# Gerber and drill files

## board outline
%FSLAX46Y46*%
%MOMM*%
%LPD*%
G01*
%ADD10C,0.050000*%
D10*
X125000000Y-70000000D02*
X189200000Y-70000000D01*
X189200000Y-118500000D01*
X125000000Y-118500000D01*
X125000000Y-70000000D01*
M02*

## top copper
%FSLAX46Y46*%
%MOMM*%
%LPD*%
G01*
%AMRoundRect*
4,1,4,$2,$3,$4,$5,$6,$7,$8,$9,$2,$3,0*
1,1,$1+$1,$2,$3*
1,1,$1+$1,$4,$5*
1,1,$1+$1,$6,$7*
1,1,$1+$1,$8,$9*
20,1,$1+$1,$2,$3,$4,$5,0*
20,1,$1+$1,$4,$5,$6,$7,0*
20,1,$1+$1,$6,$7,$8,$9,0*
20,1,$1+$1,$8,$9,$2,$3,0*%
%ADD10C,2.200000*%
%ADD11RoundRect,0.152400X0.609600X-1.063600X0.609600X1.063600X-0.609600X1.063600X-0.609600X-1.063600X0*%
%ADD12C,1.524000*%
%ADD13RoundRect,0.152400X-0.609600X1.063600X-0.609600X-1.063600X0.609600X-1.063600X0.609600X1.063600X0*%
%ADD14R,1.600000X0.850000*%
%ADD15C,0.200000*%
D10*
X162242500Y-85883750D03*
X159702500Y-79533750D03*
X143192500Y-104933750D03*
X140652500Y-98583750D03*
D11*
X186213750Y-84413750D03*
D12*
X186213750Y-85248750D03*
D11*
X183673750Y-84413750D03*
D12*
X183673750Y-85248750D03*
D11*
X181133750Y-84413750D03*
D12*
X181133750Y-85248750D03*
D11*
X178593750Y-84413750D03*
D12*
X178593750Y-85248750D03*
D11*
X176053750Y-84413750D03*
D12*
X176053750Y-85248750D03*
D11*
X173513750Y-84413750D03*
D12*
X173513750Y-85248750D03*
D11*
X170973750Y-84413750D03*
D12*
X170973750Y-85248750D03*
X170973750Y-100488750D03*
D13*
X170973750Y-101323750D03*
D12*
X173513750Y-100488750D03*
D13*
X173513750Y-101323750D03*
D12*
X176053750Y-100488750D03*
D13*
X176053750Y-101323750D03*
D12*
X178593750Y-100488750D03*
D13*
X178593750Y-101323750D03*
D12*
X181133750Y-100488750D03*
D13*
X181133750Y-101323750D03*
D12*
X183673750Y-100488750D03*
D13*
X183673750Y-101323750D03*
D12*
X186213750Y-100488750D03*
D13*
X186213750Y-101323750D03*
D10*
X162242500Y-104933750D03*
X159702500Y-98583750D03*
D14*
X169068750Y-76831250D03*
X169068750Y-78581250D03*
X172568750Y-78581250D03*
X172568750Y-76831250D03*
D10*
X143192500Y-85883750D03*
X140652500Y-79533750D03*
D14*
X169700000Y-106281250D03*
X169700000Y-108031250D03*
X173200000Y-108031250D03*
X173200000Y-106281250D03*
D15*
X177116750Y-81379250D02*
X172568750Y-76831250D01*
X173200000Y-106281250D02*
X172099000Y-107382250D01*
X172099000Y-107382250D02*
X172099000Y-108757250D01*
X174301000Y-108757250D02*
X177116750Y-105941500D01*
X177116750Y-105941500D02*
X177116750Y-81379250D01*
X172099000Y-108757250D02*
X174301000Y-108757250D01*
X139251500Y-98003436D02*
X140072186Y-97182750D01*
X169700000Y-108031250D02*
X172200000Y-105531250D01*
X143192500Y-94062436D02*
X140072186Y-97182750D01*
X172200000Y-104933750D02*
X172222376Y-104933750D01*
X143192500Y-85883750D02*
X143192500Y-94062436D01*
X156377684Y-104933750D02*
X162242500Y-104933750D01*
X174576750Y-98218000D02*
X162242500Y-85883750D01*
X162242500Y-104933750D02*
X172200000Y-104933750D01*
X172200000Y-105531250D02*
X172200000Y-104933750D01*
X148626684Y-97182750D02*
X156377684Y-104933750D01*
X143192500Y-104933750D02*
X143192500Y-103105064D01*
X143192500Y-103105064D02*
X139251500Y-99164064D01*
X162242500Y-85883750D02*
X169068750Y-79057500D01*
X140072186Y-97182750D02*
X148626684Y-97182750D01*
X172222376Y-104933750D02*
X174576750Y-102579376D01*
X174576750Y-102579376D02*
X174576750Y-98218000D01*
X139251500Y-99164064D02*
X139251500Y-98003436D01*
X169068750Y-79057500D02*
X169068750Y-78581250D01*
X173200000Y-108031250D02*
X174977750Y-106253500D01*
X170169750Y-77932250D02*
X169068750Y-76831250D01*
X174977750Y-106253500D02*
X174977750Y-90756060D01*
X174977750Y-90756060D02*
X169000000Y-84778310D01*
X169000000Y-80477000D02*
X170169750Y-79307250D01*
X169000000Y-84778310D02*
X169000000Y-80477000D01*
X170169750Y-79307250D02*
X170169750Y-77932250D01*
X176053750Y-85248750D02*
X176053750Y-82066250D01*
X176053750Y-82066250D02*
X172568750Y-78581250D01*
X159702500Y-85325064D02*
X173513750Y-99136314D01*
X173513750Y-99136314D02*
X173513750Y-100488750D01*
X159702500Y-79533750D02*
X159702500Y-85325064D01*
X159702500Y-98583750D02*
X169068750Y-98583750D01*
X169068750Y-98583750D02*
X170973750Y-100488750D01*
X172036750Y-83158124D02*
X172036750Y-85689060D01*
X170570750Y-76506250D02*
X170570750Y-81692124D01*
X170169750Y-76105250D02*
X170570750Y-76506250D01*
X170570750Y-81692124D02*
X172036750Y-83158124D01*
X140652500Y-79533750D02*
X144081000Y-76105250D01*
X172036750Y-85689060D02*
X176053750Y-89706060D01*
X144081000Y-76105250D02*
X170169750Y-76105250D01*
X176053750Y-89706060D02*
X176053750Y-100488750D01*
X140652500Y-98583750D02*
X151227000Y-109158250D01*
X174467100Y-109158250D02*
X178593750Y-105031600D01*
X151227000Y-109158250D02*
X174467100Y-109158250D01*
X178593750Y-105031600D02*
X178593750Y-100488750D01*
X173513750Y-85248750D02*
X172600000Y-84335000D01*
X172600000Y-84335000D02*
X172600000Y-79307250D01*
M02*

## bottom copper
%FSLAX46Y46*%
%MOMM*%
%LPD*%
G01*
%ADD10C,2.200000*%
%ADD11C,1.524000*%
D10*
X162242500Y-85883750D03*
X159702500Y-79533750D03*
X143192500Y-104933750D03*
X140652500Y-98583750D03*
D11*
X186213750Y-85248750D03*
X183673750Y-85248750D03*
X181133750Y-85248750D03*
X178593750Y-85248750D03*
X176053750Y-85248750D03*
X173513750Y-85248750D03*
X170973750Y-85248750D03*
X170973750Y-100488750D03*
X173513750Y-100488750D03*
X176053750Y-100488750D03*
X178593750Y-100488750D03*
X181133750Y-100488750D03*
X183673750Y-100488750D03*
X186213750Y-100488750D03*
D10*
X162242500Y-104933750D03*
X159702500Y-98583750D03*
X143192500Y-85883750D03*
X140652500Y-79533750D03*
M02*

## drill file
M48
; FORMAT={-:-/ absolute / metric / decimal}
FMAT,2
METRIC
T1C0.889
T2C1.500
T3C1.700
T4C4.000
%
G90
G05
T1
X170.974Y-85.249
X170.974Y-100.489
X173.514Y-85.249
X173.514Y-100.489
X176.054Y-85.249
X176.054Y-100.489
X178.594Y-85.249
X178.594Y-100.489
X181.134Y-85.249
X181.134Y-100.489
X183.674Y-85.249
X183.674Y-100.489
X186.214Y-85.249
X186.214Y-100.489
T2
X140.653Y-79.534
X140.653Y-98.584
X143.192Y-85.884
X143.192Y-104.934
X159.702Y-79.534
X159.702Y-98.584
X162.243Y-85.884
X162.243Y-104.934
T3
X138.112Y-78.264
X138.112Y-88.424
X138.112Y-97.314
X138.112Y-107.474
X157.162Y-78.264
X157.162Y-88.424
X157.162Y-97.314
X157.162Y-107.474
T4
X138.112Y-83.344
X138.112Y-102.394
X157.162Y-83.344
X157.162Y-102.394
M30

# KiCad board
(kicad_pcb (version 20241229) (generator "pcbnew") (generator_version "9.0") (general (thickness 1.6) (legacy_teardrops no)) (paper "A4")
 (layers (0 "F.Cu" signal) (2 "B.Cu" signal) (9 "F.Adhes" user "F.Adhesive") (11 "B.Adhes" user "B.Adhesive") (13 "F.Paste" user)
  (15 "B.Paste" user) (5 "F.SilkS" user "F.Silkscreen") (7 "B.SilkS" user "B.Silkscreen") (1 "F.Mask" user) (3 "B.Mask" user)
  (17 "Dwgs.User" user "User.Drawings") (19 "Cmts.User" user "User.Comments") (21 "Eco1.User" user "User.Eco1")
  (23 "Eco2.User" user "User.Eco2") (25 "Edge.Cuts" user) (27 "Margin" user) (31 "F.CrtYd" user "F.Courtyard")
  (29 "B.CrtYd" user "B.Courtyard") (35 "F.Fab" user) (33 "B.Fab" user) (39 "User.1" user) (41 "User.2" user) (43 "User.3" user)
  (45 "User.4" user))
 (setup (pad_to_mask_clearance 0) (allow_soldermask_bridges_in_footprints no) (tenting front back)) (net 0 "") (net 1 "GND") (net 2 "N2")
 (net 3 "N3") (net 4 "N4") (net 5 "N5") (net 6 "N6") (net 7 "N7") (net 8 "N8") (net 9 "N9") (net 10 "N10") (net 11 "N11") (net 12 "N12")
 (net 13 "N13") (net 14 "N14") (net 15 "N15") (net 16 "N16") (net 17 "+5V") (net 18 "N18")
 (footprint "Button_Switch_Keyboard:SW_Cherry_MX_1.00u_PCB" (layer "F.Cu") (at 162.2425 85.88375 -90)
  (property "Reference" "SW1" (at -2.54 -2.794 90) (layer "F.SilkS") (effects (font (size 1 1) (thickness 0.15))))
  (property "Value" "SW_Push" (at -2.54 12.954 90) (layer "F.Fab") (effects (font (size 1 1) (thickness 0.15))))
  (pad "" np_thru_hole circle (at -7.62 5.08 270) (size 1.7 1.7) (drill 1.7) (layers "*.Cu" "*.Mask"))
  (pad "" np_thru_hole circle (at -2.54 5.08 270) (size 4 4) (drill 4) (layers "*.Cu" "*.Mask"))
  (pad "" np_thru_hole circle (at 2.54 5.08 270) (size 1.7 1.7) (drill 1.7) (layers "*.Cu" "*.Mask"))
  (pad "1" thru_hole circle (at 0 0 270) (size 2.2 2.2) (drill 1.5) (layers "*.Cu" "*.Mask") (remove_unused_layers no) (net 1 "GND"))
  (pad "2" thru_hole circle (at -6.35 2.54 270) (size 2.2 2.2) (drill 1.5) (layers "*.Cu" "*.Mask") (remove_unused_layers no) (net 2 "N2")))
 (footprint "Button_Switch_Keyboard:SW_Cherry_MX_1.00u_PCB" (layer "F.Cu") (at 143.1925 104.93375 -90)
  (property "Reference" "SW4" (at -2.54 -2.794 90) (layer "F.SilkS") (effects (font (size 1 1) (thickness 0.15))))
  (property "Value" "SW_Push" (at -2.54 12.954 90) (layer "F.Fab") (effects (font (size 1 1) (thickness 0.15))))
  (pad "" np_thru_hole circle (at -7.62 5.08 270) (size 1.7 1.7) (drill 1.7) (layers "*.Cu" "*.Mask"))
  (pad "" np_thru_hole circle (at -2.54 5.08 270) (size 4 4) (drill 4) (layers "*.Cu" "*.Mask"))
  (pad "" np_thru_hole circle (at 2.54 5.08 270) (size 1.7 1.7) (drill 1.7) (layers "*.Cu" "*.Mask"))
  (pad "1" thru_hole circle (at 0 0 270) (size 2.2 2.2) (drill 1.5) (layers "*.Cu" "*.Mask") (remove_unused_layers no) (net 1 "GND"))
  (pad "2" thru_hole circle (at -6.35 2.54 270) (size 2.2 2.2) (drill 1.5) (layers "*.Cu" "*.Mask") (remove_unused_layers no) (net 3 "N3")))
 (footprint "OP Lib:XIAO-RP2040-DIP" (layer "F.Cu") (at 178.59375 92.86875 -90)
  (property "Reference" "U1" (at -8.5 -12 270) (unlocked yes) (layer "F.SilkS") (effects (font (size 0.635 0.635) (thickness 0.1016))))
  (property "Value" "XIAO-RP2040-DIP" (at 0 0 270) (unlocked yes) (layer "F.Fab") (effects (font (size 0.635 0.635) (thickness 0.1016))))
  (pad "1" smd roundrect (at -8.455 -7.62 90) (size 2.432 1.524) (layers "F.Cu" "F.Mask") (roundrect_rratio 0.1) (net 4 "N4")
   (thermal_bridge_angle 45))
  (pad "1" thru_hole circle (at -7.62 -7.62 90) (size 1.524 1.524) (drill 0.889) (layers "*.Cu" "*.Mask") (remove_unused_layers no)
   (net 4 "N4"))
  (pad "2" smd roundrect (at -8.455 -5.08 90) (size 2.432 1.524) (layers "F.Cu" "F.Mask") (roundrect_rratio 0.1) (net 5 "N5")
   (thermal_bridge_angle 45))
  (pad "2" thru_hole circle (at -7.62 -5.08 90) (size 1.524 1.524) (drill 0.889) (layers "*.Cu" "*.Mask") (remove_unused_layers no)
   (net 5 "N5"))
  (pad "3" smd roundrect (at -8.455 -2.54 90) (size 2.432 1.524) (layers "F.Cu" "F.Mask") (roundrect_rratio 0.1) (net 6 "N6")
   (thermal_bridge_angle 45))
  (pad "3" thru_hole circle (at -7.62 -2.54 90) (size 1.524 1.524) (drill 0.889) (layers "*.Cu" "*.Mask") (remove_unused_layers no)
   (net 6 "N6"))
  (pad "4" smd roundrect (at -8.455 0 90) (size 2.432 1.524) (layers "F.Cu" "F.Mask") (roundrect_rratio 0.1) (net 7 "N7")
   (thermal_bridge_angle 45))
  (pad "4" thru_hole circle (at -7.62 0 90) (size 1.524 1.524) (drill 0.889) (layers "*.Cu" "*.Mask") (remove_unused_layers no) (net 7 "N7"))
  (pad "5" smd roundrect (at -8.455 2.54 90) (size 2.432 1.524) (layers "F.Cu" "F.Mask") (roundrect_rratio 0.1) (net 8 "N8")
   (thermal_bridge_angle 45))
  (pad "5" thru_hole circle (at -7.62 2.54 90) (size 1.524 1.524) (drill 0.889) (layers "*.Cu" "*.Mask") (remove_unused_layers no)
   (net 8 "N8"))
  (pad "6" smd roundrect (at -8.455 5.08 90) (size 2.432 1.524) (layers "F.Cu" "F.Mask") (roundrect_rratio 0.1) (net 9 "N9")
   (thermal_bridge_angle 45))
  (pad "6" thru_hole circle (at -7.62 5.08 90) (size 1.524 1.524) (drill 0.889) (layers "*.Cu" "*.Mask") (remove_unused_layers no)
   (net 9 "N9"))
  (pad "7" smd roundrect (at -8.455 7.62 90) (size 2.432 1.524) (layers "F.Cu" "F.Mask") (roundrect_rratio 0.1) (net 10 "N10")
   (thermal_bridge_angle 45))
  (pad "7" thru_hole circle (at -7.62 7.62 90) (size 1.524 1.524) (drill 0.889) (layers "*.Cu" "*.Mask") (remove_unused_layers no)
   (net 10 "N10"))
  (pad "8" thru_hole circle (at 7.62 7.62 270) (size 1.524 1.524) (drill 0.889) (layers "*.Cu" "*.Mask") (remove_unused_layers no)
   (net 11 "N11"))
  (pad "8" smd roundrect (at 8.455 7.62 270) (size 2.432 1.524) (layers "F.Cu" "F.Mask") (roundrect_rratio 0.1) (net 11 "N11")
   (thermal_bridge_angle 45))
  (pad "9" thru_hole circle (at 7.62 5.08 270) (size 1.524 1.524) (drill 0.889) (layers "*.Cu" "*.Mask") (remove_unused_layers no)
   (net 2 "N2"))
  (pad "9" smd roundrect (at 8.455 5.08 270) (size 2.432 1.524) (layers "F.Cu" "F.Mask") (roundrect_rratio 0.1) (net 2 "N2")
   (thermal_bridge_angle 45))
  (pad "10" thru_hole circle (at 7.62 2.54 270) (size 1.524 1.524) (drill 0.889) (layers "*.Cu" "*.Mask") (remove_unused_layers no)
   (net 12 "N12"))
  (pad "10" smd roundrect (at 8.455 2.54 270) (size 2.432 1.524) (layers "F.Cu" "F.Mask") (roundrect_rratio 0.1) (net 12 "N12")
   (thermal_bridge_angle 45))
  (pad "11" thru_hole circle (at 7.62 0 270) (size 1.524 1.524) (drill 0.889) (layers "*.Cu" "*.Mask") (remove_unused_layers no)
   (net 3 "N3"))
  (pad "11" smd roundrect (at 8.455 0 270) (size 2.432 1.524) (layers "F.Cu" "F.Mask") (roundrect_rratio 0.1) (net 3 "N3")
   (thermal_bridge_angle 45))
  (pad "12" thru_hole circle (at 7.62 -2.54 270) (size 1.524 1.524) (drill 0.889) (layers "*.Cu" "*.Mask") (remove_unused_layers no)
   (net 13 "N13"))
  (pad "12" smd roundrect (at 8.455 -2.54 270) (size 2.432 1.524) (layers "F.Cu" "F.Mask") (roundrect_rratio 0.1) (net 13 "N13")
   (thermal_bridge_angle 45))
  (pad "13" thru_hole circle (at 7.62 -5.08 270) (size 1.524 1.524) (drill 0.889) (layers "*.Cu" "*.Mask") (remove_unused_layers no)
   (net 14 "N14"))
  (pad "13" smd roundrect (at 8.455 -5.08 270) (size 2.432 1.524) (layers "F.Cu" "F.Mask") (roundrect_rratio 0.1) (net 14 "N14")
   (thermal_bridge_angle 45))
  (pad "14" thru_hole circle (at 7.62 -7.62 270) (size 1.524 1.524) (drill 0.889) (layers "*.Cu" "*.Mask") (remove_unused_layers no)
   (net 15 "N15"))
  (pad "14" smd roundrect (at 8.455 -7.62 270) (size 2.432 1.524) (layers "F.Cu" "F.Mask") (roundrect_rratio 0.1) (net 15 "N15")
   (thermal_bridge_angle 45)))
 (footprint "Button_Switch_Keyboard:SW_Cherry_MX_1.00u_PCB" (layer "F.Cu") (at 162.2425 104.93375 -90)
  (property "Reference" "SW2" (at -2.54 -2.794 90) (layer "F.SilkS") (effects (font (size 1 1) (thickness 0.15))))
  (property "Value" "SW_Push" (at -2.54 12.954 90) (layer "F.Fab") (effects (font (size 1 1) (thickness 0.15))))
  (pad "" np_thru_hole circle (at -7.62 5.08 270) (size 1.7 1.7) (drill 1.7) (layers "*.Cu" "*.Mask"))
  (pad "" np_thru_hole circle (at -2.54 5.08 270) (size 4 4) (drill 4) (layers "*.Cu" "*.Mask"))
  (pad "" np_thru_hole circle (at 2.54 5.08 270) (size 1.7 1.7) (drill 1.7) (layers "*.Cu" "*.Mask"))
  (pad "1" thru_hole circle (at 0 0 270) (size 2.2 2.2) (drill 1.5) (layers "*.Cu" "*.Mask") (remove_unused_layers no) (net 1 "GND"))
  (pad "2" thru_hole circle (at -6.35 2.54 270) (size 2.2 2.2) (drill 1.5) (layers "*.Cu" "*.Mask") (remove_unused_layers no) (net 11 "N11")))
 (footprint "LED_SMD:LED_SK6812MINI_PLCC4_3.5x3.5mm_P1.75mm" (layer "F.Cu") (at 170.81875 77.70625)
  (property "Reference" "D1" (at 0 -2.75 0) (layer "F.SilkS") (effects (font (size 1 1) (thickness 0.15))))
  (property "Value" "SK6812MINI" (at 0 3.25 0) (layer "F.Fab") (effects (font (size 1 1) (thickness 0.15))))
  (pad "1" smd rect (at -1.75 -0.875) (size 1.6 0.85) (layers "F.Cu" "F.Mask" "F.Paste") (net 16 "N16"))
  (pad "2" smd rect (at -1.75 0.875) (size 1.6 0.85) (layers "F.Cu" "F.Mask" "F.Paste") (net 1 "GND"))
  (pad "3" smd rect (at 1.75 0.875) (size 1.6 0.85) (layers "F.Cu" "F.Mask" "F.Paste") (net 8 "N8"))
  (pad "4" smd rect (at 1.75 -0.875) (size 1.6 0.85) (layers "F.Cu" "F.Mask" "F.Paste") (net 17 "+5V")))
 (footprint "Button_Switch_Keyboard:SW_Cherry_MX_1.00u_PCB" (layer "F.Cu") (at 143.1925 85.88375 -90)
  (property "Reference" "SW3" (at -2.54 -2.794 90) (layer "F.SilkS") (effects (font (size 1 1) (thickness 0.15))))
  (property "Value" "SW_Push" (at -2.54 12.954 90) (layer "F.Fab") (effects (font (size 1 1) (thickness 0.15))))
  (pad "" np_thru_hole circle (at -7.62 5.08 270) (size 1.7 1.7) (drill 1.7) (layers "*.Cu" "*.Mask"))
  (pad "" np_thru_hole circle (at -2.54 5.08 270) (size 4 4) (drill 4) (layers "*.Cu" "*.Mask"))
  (pad "" np_thru_hole circle (at 2.54 5.08 270) (size 1.7 1.7) (drill 1.7) (layers "*.Cu" "*.Mask"))
  (pad "1" thru_hole circle (at 0 0 270) (size 2.2 2.2) (drill 1.5) (layers "*.Cu" "*.Mask") (remove_unused_layers no) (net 1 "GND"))
  (pad "2" thru_hole circle (at -6.35 2.54 270) (size 2.2 2.2) (drill 1.5) (layers "*.Cu" "*.Mask") (remove_unused_layers no) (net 12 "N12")))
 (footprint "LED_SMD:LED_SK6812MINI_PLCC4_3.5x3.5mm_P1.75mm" (layer "F.Cu") (at 171.45 107.15625)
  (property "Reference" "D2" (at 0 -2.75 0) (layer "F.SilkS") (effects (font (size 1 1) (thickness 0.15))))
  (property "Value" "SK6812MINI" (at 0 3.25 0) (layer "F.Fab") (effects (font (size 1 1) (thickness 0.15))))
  (pad "1" smd rect (at -1.75 -0.875) (size 1.6 0.85) (layers "F.Cu" "F.Mask" "F.Paste") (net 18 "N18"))
  (pad "2" smd rect (at -1.75 0.875) (size 1.6 0.85) (layers "F.Cu" "F.Mask" "F.Paste") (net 1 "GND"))
  (pad "3" smd rect (at 1.75 0.875) (size 1.6 0.85) (layers "F.Cu" "F.Mask" "F.Paste") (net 16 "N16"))
  (pad "4" smd rect (at 1.75 -0.875) (size 1.6 0.85) (layers "F.Cu" "F.Mask" "F.Paste") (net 17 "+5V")))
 (gr_rect (start 125 70) (end 189.2 118.5) (stroke (width 0.05) (type default)) (fill no) (layer "Edge.Cuts"))
 (segment (start 177.11675 81.37925) (end 172.56875 76.83125) (width 0.2) (layer "F.Cu") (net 17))
 (segment (start 173.2 106.28125) (end 172.099 107.38225) (width 0.2) (layer "F.Cu") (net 17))
 (segment (start 172.099 107.38225) (end 172.099 108.75725) (width 0.2) (layer "F.Cu") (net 17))
 (segment (start 174.301 108.75725) (end 177.11675 105.9415) (width 0.2) (layer "F.Cu") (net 17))
 (segment (start 177.11675 105.9415) (end 177.11675 81.37925) (width 0.2) (layer "F.Cu") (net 17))
 (segment (start 172.099 108.75725) (end 174.301 108.75725) (width 0.2) (layer "F.Cu") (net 17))
 (segment (start 139.2515 98.003436) (end 140.072186 97.18275) (width 0.2) (layer "F.Cu") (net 1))
 (segment (start 169.7 108.03125) (end 172.2 105.53125) (width 0.2) (layer "F.Cu") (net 1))
 (segment (start 143.1925 94.062436) (end 140.072186 97.18275) (width 0.2) (layer "F.Cu") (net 1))
 (segment (start 172.2 104.93375) (end 172.222376 104.93375) (width 0.2) (layer "F.Cu") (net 1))
 (segment (start 143.1925 85.88375) (end 143.1925 94.062436) (width 0.2) (layer "F.Cu") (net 1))
 (segment (start 156.377684 104.93375) (end 162.2425 104.93375) (width 0.2) (layer "F.Cu") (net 1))
 (segment (start 174.57675 98.218) (end 162.2425 85.88375) (width 0.2) (layer "F.Cu") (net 1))
 (segment (start 162.2425 104.93375) (end 172.2 104.93375) (width 0.2) (layer "F.Cu") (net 1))
 (segment (start 172.2 105.53125) (end 172.2 104.93375) (width 0.2) (layer "F.Cu") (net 1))
 (segment (start 148.626684 97.18275) (end 156.377684 104.93375) (width 0.2) (layer "F.Cu") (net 1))
 (segment (start 143.1925 104.93375) (end 143.1925 103.105064) (width 0.2) (layer "F.Cu") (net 1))
 (segment (start 143.1925 103.105064) (end 139.2515 99.164064) (width 0.2) (layer "F.Cu") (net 1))
 (segment (start 162.2425 85.88375) (end 169.06875 79.0575) (width 0.2) (layer "F.Cu") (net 1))
 (segment (start 140.072186 97.18275) (end 148.626684 97.18275) (width 0.2) (layer "F.Cu") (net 1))
 (segment (start 172.222376 104.93375) (end 174.57675 102.579376) (width 0.2) (layer "F.Cu") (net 1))
 (segment (start 174.57675 102.579376) (end 174.57675 98.218) (width 0.2) (layer "F.Cu") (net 1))
 (segment (start 139.2515 99.164064) (end 139.2515 98.003436) (width 0.2) (layer "F.Cu") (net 1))
 (segment (start 169.06875 79.0575) (end 169.06875 78.58125) (width 0.2) (layer "F.Cu") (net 1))
 (segment (start 173.2 108.03125) (end 174.97775 106.2535) (width 0.2) (layer "F.Cu") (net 16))
 (segment (start 170.16975 77.93225) (end 169.06875 76.83125) (width 0.2) (layer "F.Cu") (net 16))
 (segment (start 174.97775 106.2535) (end 174.97775 90.75606) (width 0.2) (layer "F.Cu") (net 16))
 (segment (start 174.97775 90.75606) (end 169 84.77831) (width 0.2) (layer "F.Cu") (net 16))
 (segment (start 169 80.477) (end 170.16975 79.30725) (width 0.2) (layer "F.Cu") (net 16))
 (segment (start 169 84.77831) (end 169 80.477) (width 0.2) (layer "F.Cu") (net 16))
 (segment (start 170.16975 79.30725) (end 170.16975 77.93225) (width 0.2) (layer "F.Cu") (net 16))
 (segment (start 176.05375 85.24875) (end 176.05375 82.06625) (width 0.2) (layer "F.Cu") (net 8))
 (segment (start 176.05375 82.06625) (end 172.56875 78.58125) (width 0.2) (layer "F.Cu") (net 8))
 (segment (start 159.7025 85.325064) (end 173.51375 99.136314) (width 0.2) (layer "F.Cu") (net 2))
 (segment (start 173.51375 99.136314) (end 173.51375 100.48875) (width 0.2) (layer "F.Cu") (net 2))
 (segment (start 159.7025 79.53375) (end 159.7025 85.325064) (width 0.2) (layer "F.Cu") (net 2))
 (segment (start 159.7025 98.58375) (end 169.06875 98.58375) (width 0.2) (layer "F.Cu") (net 11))
 (segment (start 169.06875 98.58375) (end 170.97375 100.48875) (width 0.2) (layer "F.Cu") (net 11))
 (segment (start 172.03675 83.158124) (end 172.03675 85.68906) (width 0.2) (layer "F.Cu") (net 12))
 (segment (start 170.57075 76.50625) (end 170.57075 81.692124) (width 0.2) (layer "F.Cu") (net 12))
 (segment (start 170.16975 76.10525) (end 170.57075 76.50625) (width 0.2) (layer "F.Cu") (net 12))
 (segment (start 170.57075 81.692124) (end 172.03675 83.158124) (width 0.2) (layer "F.Cu") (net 12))
 (segment (start 140.6525 79.53375) (end 144.081 76.10525) (width 0.2) (layer "F.Cu") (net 12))
 (segment (start 172.03675 85.68906) (end 176.05375 89.70606) (width 0.2) (layer "F.Cu") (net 12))
 (segment (start 144.081 76.10525) (end 170.16975 76.10525) (width 0.2) (layer "F.Cu") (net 12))
 (segment (start 176.05375 89.70606) (end 176.05375 100.48875) (width 0.2) (layer "F.Cu") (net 12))
 (segment (start 140.6525 98.58375) (end 151.227 109.15825) (width 0.2) (layer "F.Cu") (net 3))
 (segment (start 174.4671 109.15825) (end 178.59375 105.0316) (width 0.2) (layer "F.Cu") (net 3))
 (segment (start 151.227 109.15825) (end 174.4671 109.15825) (width 0.2) (layer "F.Cu") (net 3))
 (segment (start 178.59375 105.0316) (end 178.59375 100.48875) (width 0.2) (layer "F.Cu") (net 3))
 (segment (start 173.51375 85.24875) (end 172.6 84.335) (width 0.2) (layer "F.Cu") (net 9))
 (segment (start 172.6 84.335) (end 172.6 79.30725) (width 0.2) (layer "F.Cu") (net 9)))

